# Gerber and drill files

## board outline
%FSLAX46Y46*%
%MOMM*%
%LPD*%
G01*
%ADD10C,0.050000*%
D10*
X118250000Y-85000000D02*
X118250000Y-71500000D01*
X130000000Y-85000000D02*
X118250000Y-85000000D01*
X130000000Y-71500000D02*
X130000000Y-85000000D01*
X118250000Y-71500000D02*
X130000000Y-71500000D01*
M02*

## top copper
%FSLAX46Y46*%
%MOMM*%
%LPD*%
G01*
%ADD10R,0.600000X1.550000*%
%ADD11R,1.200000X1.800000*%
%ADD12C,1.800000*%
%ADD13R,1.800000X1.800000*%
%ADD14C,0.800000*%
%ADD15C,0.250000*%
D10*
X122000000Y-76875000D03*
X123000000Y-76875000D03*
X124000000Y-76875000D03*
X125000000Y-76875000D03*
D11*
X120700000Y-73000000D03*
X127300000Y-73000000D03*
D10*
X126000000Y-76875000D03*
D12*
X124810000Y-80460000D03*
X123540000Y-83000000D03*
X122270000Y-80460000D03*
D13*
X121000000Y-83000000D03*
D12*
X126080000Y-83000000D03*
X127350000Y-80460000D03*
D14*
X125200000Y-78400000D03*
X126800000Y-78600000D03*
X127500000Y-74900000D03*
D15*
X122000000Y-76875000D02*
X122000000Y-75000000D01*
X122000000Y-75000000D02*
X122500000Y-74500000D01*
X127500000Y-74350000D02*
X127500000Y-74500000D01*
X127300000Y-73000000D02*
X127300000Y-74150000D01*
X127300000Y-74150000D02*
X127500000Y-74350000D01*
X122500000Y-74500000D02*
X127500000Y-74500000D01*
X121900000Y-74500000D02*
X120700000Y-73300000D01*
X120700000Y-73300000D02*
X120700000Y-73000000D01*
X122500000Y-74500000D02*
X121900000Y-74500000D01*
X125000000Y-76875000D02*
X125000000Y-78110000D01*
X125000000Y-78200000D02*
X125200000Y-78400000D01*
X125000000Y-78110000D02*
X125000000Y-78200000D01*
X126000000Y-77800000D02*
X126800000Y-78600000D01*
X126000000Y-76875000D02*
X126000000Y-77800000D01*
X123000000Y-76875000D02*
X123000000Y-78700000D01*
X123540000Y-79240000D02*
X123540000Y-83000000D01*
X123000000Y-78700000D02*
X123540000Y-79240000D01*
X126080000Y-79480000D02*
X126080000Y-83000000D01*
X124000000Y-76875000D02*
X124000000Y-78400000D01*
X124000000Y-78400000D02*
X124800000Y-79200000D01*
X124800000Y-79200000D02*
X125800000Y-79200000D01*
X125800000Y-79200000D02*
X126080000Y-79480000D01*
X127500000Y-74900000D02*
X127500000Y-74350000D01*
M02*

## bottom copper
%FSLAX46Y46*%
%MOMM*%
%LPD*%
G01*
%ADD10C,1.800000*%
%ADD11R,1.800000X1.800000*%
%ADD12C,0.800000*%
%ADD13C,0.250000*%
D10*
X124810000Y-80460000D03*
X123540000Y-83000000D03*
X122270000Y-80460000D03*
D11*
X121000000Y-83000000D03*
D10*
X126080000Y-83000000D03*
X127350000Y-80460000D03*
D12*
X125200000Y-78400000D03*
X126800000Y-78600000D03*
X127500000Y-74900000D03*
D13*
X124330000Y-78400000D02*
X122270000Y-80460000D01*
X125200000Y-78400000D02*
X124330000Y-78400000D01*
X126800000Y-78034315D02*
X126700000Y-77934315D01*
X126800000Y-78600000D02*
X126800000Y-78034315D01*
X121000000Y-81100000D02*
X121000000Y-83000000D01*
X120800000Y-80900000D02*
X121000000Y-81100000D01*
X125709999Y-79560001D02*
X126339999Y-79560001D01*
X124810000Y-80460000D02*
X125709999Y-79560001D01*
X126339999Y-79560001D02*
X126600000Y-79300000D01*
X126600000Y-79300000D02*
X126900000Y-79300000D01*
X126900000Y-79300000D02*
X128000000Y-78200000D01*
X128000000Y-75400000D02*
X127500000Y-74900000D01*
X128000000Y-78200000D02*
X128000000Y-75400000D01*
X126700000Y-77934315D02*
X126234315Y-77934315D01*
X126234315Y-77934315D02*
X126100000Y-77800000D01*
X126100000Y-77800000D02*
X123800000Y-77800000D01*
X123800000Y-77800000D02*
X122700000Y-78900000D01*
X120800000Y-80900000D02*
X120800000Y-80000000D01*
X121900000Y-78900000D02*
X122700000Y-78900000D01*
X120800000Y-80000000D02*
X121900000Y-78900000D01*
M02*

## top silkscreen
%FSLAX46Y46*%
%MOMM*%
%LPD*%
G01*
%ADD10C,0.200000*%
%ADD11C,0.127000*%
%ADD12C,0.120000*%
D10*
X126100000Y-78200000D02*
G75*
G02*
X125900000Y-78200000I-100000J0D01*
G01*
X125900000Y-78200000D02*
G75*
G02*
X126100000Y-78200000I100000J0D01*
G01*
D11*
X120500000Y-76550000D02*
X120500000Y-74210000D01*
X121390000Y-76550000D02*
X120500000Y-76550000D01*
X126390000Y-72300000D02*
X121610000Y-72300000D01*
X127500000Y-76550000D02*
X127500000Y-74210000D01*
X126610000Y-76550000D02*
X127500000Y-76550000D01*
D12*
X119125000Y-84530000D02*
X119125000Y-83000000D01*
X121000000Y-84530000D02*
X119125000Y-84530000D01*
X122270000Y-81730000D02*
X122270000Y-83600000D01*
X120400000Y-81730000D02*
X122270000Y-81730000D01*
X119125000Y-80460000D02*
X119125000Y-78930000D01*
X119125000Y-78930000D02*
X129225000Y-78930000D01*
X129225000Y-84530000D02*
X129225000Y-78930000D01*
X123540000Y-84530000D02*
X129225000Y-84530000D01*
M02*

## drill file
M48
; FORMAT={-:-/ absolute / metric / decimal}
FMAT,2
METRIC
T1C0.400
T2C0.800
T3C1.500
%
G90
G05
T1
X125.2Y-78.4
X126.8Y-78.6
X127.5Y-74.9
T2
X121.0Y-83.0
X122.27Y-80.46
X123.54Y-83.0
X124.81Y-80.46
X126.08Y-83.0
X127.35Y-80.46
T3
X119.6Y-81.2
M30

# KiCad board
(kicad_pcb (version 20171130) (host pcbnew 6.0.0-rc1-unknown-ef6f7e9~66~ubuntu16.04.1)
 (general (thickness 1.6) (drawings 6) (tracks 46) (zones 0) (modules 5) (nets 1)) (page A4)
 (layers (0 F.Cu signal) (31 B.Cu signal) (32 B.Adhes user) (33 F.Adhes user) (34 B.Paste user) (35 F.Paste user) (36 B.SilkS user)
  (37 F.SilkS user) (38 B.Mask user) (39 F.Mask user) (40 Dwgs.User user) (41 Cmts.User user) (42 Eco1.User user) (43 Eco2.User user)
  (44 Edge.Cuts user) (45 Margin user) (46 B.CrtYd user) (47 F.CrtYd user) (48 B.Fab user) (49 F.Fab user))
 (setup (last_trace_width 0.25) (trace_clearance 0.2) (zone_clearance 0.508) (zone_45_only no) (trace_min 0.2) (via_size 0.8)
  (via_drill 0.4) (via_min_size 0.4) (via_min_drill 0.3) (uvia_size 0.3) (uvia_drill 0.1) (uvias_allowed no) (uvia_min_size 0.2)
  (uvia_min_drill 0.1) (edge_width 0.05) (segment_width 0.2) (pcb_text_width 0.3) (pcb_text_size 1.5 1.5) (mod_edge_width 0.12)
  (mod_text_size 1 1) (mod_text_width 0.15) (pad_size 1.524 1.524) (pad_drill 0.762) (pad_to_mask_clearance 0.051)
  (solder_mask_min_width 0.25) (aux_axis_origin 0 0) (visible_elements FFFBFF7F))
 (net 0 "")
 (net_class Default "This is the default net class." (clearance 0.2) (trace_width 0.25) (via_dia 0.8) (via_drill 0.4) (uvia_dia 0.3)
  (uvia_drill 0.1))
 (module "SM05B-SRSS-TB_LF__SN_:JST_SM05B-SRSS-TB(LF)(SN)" (layer F.Cu) (at 124 73 180)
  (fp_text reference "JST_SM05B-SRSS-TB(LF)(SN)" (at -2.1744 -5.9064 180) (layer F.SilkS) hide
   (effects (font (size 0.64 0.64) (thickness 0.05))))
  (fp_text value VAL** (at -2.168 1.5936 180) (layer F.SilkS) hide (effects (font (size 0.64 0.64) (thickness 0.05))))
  (fp_circle (center -2 -5.2) (end -1.9 -5.2) (layer F.SilkS) (width 0.2))
  (fp_line (start 3.5 -3.55) (end 3.5 -1.21) (layer F.SilkS) (width 0.127))
  (fp_line (start 2.61 -3.55) (end 3.5 -3.55) (layer F.SilkS) (width 0.127))
  (fp_line (start -2.39 0.7) (end 2.39 0.7) (layer F.SilkS) (width 0.127))
  (fp_line (start -3.5 -3.55) (end -3.5 -1.21) (layer F.SilkS) (width 0.127))
  (fp_line (start -2.61 -3.55) (end -3.5 -3.55) (layer F.SilkS) (width 0.127))
  (pad 5 smd rect (at 2 -3.875 270) (size 1.55 0.6) (layers F.Cu F.Paste F.Mask))
  (pad 4 smd rect (at 1 -3.875 270) (size 1.55 0.6) (layers F.Cu F.Paste F.Mask))
  (pad 3 smd rect (at 0 -3.875 270) (size 1.55 0.6) (layers F.Cu F.Paste F.Mask))
  (pad 2 smd rect (at -1 -3.875 270) (size 1.55 0.6) (layers F.Cu F.Paste F.Mask))
  (pad S2 smd rect (at 3.3 0 270) (size 1.8 1.2) (layers F.Cu F.Paste F.Mask))
  (pad S1 smd rect (at -3.3 0 270) (size 1.8 1.2) (layers F.Cu F.Paste F.Mask))
  (pad 1 smd rect (at -2 -3.875 270) (size 1.55 0.6) (layers F.Cu F.Paste F.Mask)))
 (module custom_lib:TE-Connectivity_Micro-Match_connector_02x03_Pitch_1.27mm (layer F.Cu) (at 121 83 90)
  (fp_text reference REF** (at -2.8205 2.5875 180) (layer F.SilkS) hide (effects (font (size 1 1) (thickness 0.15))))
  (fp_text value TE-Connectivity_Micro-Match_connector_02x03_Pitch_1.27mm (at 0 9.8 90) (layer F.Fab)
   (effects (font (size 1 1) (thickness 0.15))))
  (fp_line (start -1.53 -1.875) (end 0 -1.875) (layer F.SilkS) (width 0.12))
  (fp_line (start -1.53 0) (end -1.53 -1.875) (layer F.SilkS) (width 0.12))
  (fp_line (start 1.27 1.27) (end -0.6 1.27) (layer F.SilkS) (width 0.12))
  (fp_line (start 1.27 -0.6) (end 1.27 1.27) (layer F.SilkS) (width 0.12))
  (fp_line (start 2.54 -1.875) (end 4.07 -1.875) (layer F.SilkS) (width 0.12))
  (fp_line (start 4.07 -1.875) (end 4.07 8.225) (layer F.SilkS) (width 0.12))
  (fp_line (start -1.53 8.225) (end 4.07 8.225) (layer F.SilkS) (width 0.12))
  (fp_line (start -1.53 2.54) (end -1.53 8.225) (layer F.SilkS) (width 0.12))
  (pad "" np_thru_hole circle (at 1.8 -1.4 90) (size 1.5001 1.5001) (drill 1.5001) (layers *.Cu *.Mask))
  (pad 4 thru_hole circle (at 2.54 3.81 90) (size 1.8 1.8) (drill 0.8001) (layers *.Cu *.Mask))
  (pad 3 thru_hole circle (at 0 2.54 90) (size 1.8 1.8) (drill 0.8001) (layers *.Cu *.Mask))
  (pad 2 thru_hole circle (at 2.54 1.27 90) (size 1.8 1.8) (drill 0.8001) (layers *.Cu *.Mask))
  (pad 1 thru_hole rect (at 0 0 90) (size 1.8 1.8) (drill 0.8001) (layers *.Cu *.Mask))
  (pad 5 thru_hole circle (at 0 5.08 90) (size 1.8 1.8) (drill 0.8001) (layers *.Cu *.Mask))
  (pad 6 thru_hole circle (at 2.54 6.35 90) (size 1.8 1.8) (drill 0.8001) (layers *.Cu *.Mask)))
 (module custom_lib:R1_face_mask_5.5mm (layer B.Cu) (at 121.4 76)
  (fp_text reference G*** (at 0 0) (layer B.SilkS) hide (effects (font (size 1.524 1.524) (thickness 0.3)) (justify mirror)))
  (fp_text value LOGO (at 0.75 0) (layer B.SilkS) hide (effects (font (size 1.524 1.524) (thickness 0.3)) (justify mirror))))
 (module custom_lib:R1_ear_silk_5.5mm (layer B.Cu) (at 121.4 76)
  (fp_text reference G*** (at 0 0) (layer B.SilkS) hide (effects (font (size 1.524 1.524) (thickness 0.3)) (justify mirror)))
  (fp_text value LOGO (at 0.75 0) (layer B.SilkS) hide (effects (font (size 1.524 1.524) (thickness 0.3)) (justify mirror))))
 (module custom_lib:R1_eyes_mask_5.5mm (layer B.Cu) (at 121.4 76)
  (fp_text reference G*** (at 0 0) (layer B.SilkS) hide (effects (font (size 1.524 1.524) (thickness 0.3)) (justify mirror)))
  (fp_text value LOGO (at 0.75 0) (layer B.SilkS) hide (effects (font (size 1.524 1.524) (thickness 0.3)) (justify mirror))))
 (gr_line (start 118.25 85) (end 118.25 71.5) (layer Edge.Cuts) (width 0.05))
 (gr_line (start 130 85) (end 118.25 85) (layer Edge.Cuts) (width 0.05))
 (gr_line (start 130 71.5) (end 130 85) (layer Edge.Cuts) (width 0.05))
 (gr_line (start 118.25 71.5) (end 130 71.5) (layer Edge.Cuts) (width 0.05))
 (segment (start 122 76.875) (end 122 75) (width 0.25) (layer F.Cu) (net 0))
 (segment (start 122 75) (end 122.5 74.5) (width 0.25) (layer F.Cu) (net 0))
 (segment (start 127.5 74.35) (end 127.5 74.5) (width 0.25) (layer F.Cu) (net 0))
 (segment (start 127.3 73) (end 127.3 74.15) (width 0.25) (layer F.Cu) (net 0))
 (segment (start 127.3 74.15) (end 127.5 74.35) (width 0.25) (layer F.Cu) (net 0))
 (segment (start 122.5 74.5) (end 127.5 74.5) (width 0.25) (layer F.Cu) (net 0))
 (segment (start 121.9 74.5) (end 120.7 73.3) (width 0.25) (layer F.Cu) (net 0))
 (segment (start 120.7 73.3) (end 120.7 73) (width 0.25) (layer F.Cu) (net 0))
 (segment (start 122.5 74.5) (end 121.9 74.5) (width 0.25) (layer F.Cu) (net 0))
 (segment (start 125 76.875) (end 125 78.11) (width 0.25) (layer F.Cu) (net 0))
 (via (at 125.2 78.4) (size 0.8) (drill 0.4) (layers F.Cu B.Cu) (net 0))
 (segment (start 125 78.2) (end 125.2 78.4) (width 0.25) (layer F.Cu) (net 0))
 (segment (start 125 78.11) (end 125 78.2) (width 0.25) (layer F.Cu) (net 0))
 (segment (start 124.33 78.4) (end 122.27 80.46) (width 0.25) (layer B.Cu) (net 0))
 (segment (start 125.2 78.4) (end 124.33 78.4) (width 0.25) (layer B.Cu) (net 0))
 (via (at 126.8 78.6) (size 0.8) (drill 0.4) (layers F.Cu B.Cu) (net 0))
 (segment (start 126 77.8) (end 126.8 78.6) (width 0.25) (layer F.Cu) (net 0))
 (segment (start 126 76.875) (end 126 77.8) (width 0.25) (layer F.Cu) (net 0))
 (segment (start 126.8 78.034315) (end 126.7 77.934315) (width 0.25) (layer B.Cu) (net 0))
 (segment (start 126.8 78.6) (end 126.8 78.034315) (width 0.25) (layer B.Cu) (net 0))
 (segment (start 121 81.1) (end 121 83) (width 0.25) (layer B.Cu) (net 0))
 (segment (start 120.8 80.9) (end 121 81.1) (width 0.25) (layer B.Cu) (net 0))
 (segment (start 123 76.875) (end 123 78.7) (width 0.25) (layer F.Cu) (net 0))
 (segment (start 123.54 79.24) (end 123.54 83) (width 0.25) (layer F.Cu) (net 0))
 (segment (start 123 78.7) (end 123.54 79.24) (width 0.25) (layer F.Cu) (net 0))
 (segment (start 126.08 79.48) (end 126.08 83) (width 0.25) (layer F.Cu) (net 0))
 (segment (start 124 76.875) (end 124 78.4) (width 0.25) (layer F.Cu) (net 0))
 (segment (start 124 78.4) (end 124.8 79.2) (width 0.25) (layer F.Cu) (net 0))
 (segment (start 124.8 79.2) (end 125.8 79.2) (width 0.25) (layer F.Cu) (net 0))
 (segment (start 125.8 79.2) (end 126.08 79.48) (width 0.25) (layer F.Cu) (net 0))
 (segment (start 125.709999 79.560001) (end 126.339999 79.560001) (width 0.25) (layer B.Cu) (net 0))
 (segment (start 124.81 80.46) (end 125.709999 79.560001) (width 0.25) (layer B.Cu) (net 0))
 (segment (start 126.339999 79.560001) (end 126.6 79.3) (width 0.25) (layer B.Cu) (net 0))
 (segment (start 126.6 79.3) (end 126.9 79.3) (width 0.25) (layer B.Cu) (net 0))
 (segment (start 126.9 79.3) (end 128 78.2) (width 0.25) (layer B.Cu) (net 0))
 (segment (start 128 75.4) (end 127.5 74.9) (width 0.25) (layer B.Cu) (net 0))
 (via (at 127.5 74.9) (size 0.8) (drill 0.4) (layers F.Cu B.Cu) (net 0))
 (segment (start 128 78.2) (end 128 75.4) (width 0.25) (layer B.Cu) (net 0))
 (segment (start 127.5 74.9) (end 127.5 74.35) (width 0.25) (layer F.Cu) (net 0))
 (segment (start 126.7 77.934315) (end 126.234315 77.934315) (width 0.25) (layer B.Cu) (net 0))
 (segment (start 126.234315 77.934315) (end 126.1 77.8) (width 0.25) (layer B.Cu) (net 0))
 (segment (start 126.1 77.8) (end 123.8 77.8) (width 0.25) (layer B.Cu) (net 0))
 (segment (start 123.8 77.8) (end 122.7 78.9) (width 0.25) (layer B.Cu) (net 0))
 (segment (start 120.8 80.9) (end 120.8 80) (width 0.25) (layer B.Cu) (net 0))
 (segment (start 121.9 78.9) (end 122.7 78.9) (width 0.25) (layer B.Cu) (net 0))
 (segment (start 120.8 80) (end 121.9 78.9) (width 0.25) (layer B.Cu) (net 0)))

